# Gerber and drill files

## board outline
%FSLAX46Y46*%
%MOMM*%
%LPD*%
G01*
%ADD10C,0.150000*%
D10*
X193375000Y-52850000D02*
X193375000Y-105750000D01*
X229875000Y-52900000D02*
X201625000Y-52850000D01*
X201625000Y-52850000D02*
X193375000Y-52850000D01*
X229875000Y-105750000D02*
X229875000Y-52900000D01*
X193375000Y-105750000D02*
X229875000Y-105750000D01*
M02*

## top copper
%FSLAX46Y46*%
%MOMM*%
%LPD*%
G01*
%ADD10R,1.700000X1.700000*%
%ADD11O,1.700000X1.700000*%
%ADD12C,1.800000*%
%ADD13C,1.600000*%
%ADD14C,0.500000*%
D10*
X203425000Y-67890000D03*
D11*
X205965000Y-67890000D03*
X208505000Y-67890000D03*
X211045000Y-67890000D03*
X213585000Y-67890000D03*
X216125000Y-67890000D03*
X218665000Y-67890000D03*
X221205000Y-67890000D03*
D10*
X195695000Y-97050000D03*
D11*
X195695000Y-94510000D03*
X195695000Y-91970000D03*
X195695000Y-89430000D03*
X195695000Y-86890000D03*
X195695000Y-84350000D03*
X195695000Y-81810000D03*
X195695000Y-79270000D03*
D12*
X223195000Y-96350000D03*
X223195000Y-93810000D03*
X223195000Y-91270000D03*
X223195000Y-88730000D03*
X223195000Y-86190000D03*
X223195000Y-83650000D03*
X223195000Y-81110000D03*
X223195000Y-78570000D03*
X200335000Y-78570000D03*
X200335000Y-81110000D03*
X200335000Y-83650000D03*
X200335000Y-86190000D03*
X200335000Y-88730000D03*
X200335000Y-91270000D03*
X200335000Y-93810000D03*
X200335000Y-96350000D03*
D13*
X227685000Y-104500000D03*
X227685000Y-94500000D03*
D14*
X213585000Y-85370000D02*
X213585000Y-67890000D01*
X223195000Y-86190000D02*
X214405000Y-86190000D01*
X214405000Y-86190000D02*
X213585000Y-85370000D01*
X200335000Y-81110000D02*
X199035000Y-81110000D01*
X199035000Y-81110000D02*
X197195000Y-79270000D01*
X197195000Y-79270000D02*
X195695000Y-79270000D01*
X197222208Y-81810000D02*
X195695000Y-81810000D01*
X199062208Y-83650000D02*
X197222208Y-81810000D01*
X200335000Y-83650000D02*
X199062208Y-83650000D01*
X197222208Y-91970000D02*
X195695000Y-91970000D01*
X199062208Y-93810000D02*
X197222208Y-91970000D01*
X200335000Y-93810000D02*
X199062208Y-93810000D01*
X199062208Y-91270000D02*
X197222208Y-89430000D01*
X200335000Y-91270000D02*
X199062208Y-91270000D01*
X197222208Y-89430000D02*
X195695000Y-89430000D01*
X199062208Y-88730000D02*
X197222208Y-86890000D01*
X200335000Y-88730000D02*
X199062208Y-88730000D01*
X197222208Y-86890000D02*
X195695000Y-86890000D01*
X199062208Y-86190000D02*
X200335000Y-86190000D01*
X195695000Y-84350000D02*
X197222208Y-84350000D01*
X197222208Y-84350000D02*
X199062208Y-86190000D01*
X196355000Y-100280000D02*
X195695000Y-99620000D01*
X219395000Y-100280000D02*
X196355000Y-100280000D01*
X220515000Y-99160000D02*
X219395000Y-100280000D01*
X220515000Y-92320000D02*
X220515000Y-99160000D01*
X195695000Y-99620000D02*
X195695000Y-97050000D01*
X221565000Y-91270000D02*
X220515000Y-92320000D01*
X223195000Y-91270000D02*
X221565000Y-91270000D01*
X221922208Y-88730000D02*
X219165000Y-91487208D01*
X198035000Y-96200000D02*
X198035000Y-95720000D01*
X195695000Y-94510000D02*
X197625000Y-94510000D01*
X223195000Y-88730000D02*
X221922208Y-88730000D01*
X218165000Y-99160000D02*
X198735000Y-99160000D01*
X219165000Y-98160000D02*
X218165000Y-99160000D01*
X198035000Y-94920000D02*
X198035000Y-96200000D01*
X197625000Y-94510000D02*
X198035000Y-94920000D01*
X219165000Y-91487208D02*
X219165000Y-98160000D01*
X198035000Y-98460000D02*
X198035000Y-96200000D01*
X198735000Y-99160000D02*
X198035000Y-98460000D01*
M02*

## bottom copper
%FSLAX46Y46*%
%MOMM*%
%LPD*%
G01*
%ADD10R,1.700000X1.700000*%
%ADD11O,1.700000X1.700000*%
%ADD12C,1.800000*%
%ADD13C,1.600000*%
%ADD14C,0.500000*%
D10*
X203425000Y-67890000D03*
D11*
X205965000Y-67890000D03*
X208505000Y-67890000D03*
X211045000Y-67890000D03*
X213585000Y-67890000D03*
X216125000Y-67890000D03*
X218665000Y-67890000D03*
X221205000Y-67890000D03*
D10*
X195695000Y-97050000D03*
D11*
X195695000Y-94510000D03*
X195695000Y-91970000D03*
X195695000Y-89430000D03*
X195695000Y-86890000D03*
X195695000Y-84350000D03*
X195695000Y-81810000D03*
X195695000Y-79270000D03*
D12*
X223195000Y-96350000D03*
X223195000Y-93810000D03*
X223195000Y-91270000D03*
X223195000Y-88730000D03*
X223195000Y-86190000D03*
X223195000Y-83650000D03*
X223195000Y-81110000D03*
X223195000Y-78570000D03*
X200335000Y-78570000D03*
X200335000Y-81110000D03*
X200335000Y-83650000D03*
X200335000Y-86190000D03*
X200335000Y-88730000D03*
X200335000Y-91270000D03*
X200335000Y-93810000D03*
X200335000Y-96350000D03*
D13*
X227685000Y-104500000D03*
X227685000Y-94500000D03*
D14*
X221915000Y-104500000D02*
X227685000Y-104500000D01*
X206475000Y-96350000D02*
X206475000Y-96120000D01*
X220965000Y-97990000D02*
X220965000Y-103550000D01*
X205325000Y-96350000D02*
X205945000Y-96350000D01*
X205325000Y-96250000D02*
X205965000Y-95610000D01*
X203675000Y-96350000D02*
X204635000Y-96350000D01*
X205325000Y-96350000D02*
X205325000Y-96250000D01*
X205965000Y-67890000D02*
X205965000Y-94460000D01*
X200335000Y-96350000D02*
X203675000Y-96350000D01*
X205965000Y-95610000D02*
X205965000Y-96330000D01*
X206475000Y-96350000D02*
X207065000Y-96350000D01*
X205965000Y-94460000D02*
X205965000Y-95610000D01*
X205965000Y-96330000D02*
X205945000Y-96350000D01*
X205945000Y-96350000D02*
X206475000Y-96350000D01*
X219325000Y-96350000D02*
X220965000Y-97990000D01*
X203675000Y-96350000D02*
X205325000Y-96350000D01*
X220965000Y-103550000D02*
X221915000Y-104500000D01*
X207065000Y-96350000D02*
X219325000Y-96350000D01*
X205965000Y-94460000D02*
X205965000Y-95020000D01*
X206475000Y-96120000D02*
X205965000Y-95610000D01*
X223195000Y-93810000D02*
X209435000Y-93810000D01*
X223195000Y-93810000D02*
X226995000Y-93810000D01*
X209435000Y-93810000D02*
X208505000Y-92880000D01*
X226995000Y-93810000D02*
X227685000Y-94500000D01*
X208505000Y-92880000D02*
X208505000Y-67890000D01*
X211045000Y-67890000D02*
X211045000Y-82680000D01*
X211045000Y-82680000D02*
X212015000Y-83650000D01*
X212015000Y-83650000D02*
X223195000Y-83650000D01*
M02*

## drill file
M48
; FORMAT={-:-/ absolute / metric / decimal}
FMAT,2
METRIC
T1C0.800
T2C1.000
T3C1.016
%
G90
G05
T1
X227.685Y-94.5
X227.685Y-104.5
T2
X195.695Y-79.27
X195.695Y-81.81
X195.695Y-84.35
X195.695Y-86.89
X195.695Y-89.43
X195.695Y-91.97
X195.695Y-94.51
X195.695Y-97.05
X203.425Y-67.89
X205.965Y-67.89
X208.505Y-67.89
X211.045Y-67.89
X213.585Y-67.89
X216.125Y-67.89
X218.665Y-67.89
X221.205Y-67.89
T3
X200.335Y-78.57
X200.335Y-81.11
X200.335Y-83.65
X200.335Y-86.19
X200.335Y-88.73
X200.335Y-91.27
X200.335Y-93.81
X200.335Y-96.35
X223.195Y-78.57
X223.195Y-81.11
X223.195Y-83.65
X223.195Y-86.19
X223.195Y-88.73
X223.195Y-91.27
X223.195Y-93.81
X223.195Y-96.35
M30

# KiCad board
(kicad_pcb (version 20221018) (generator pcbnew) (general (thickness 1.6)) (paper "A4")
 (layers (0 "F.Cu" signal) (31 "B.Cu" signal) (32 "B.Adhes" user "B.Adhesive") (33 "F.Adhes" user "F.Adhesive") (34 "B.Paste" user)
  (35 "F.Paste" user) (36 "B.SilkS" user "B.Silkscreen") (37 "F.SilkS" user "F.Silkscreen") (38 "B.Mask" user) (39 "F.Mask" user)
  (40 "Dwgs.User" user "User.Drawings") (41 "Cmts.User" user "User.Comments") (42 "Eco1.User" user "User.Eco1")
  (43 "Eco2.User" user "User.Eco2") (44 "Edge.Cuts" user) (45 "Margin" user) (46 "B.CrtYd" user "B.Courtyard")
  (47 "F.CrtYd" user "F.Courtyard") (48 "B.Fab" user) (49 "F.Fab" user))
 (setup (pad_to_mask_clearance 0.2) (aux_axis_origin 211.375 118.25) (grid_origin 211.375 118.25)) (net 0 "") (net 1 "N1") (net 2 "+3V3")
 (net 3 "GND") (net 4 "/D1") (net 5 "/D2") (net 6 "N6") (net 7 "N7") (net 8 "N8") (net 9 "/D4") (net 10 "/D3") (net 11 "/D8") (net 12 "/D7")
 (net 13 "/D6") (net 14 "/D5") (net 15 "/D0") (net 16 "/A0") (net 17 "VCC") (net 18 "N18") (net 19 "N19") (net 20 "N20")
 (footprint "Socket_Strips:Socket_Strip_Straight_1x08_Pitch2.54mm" (layer "F.Cu") (at 203.425 67.89 90)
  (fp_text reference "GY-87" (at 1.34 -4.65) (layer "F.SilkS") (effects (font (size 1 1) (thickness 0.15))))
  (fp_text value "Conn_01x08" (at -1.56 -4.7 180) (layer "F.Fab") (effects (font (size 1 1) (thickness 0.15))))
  (pad "1" thru_hole rect (at 0 0 90) (size 1.7 1.7) (drill 1) (layers "*.Cu" "*.Mask") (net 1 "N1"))
  (pad "2" thru_hole oval (at 0 2.54 90) (size 1.7 1.7) (drill 1) (layers "*.Cu" "*.Mask") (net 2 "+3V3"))
  (pad "3" thru_hole oval (at 0 5.08 90) (size 1.7 1.7) (drill 1) (layers "*.Cu" "*.Mask") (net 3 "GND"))
  (pad "4" thru_hole oval (at 0 7.62 90) (size 1.7 1.7) (drill 1) (layers "*.Cu" "*.Mask") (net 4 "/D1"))
  (pad "5" thru_hole oval (at 0 10.16 90) (size 1.7 1.7) (drill 1) (layers "*.Cu" "*.Mask") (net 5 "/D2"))
  (pad "6" thru_hole oval (at 0 12.7 90) (size 1.7 1.7) (drill 1) (layers "*.Cu" "*.Mask") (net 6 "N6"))
  (pad "7" thru_hole oval (at 0 15.24 90) (size 1.7 1.7) (drill 1) (layers "*.Cu" "*.Mask") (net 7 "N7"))
  (pad "8" thru_hole oval (at 0 17.78 90) (size 1.7 1.7) (drill 1) (layers "*.Cu" "*.Mask") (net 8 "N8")))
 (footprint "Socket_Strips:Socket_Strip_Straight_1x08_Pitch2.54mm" (layer "F.Cu") (at 195.695 97.05 180)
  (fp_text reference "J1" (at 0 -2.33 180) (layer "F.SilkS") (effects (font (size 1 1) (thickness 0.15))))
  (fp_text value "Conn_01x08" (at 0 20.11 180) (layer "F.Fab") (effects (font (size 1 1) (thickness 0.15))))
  (pad "1" thru_hole rect (at 0 0 180) (size 1.7 1.7) (drill 1) (layers "*.Cu" "*.Mask") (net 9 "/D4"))
  (pad "2" thru_hole oval (at 0 2.54 180) (size 1.7 1.7) (drill 1) (layers "*.Cu" "*.Mask") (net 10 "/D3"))
  (pad "3" thru_hole oval (at 0 5.08 180) (size 1.7 1.7) (drill 1) (layers "*.Cu" "*.Mask") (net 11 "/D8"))
  (pad "4" thru_hole oval (at 0 7.62 180) (size 1.7 1.7) (drill 1) (layers "*.Cu" "*.Mask") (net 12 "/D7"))
  (pad "5" thru_hole oval (at 0 10.16 180) (size 1.7 1.7) (drill 1) (layers "*.Cu" "*.Mask") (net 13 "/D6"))
  (pad "6" thru_hole oval (at 0 12.7 180) (size 1.7 1.7) (drill 1) (layers "*.Cu" "*.Mask") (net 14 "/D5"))
  (pad "7" thru_hole oval (at 0 15.24 180) (size 1.7 1.7) (drill 1) (layers "*.Cu" "*.Mask") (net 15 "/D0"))
  (pad "8" thru_hole oval (at 0 17.78 180) (size 1.7 1.7) (drill 1) (layers "*.Cu" "*.Mask") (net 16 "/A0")))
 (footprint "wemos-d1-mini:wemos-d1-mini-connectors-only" (layer "F.Cu") (at 211.765 87.46 90)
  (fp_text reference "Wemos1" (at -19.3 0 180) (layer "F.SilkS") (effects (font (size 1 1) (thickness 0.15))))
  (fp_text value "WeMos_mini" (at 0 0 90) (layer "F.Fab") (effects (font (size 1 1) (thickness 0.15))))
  (pad "1" thru_hole circle (at -8.89 11.43 90) (size 1.8 1.8) (drill 1.016) (layers "*.Cu" "*.Mask") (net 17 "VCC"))
  (pad "2" thru_hole circle (at -6.35 11.43 90) (size 1.8 1.8) (drill 1.016) (layers "*.Cu" "*.Mask") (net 3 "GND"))
  (pad "3" thru_hole circle (at -3.81 11.43 90) (size 1.8 1.8) (drill 1.016) (layers "*.Cu" "*.Mask") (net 9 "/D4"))
  (pad "4" thru_hole circle (at -1.27 11.43 90) (size 1.8 1.8) (drill 1.016) (layers "*.Cu" "*.Mask") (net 10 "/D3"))
  (pad "5" thru_hole circle (at 1.27 11.43 90) (size 1.8 1.8) (drill 1.016) (layers "*.Cu" "*.Mask") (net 5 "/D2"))
  (pad "6" thru_hole circle (at 3.81 11.43 90) (size 1.8 1.8) (drill 1.016) (layers "*.Cu" "*.Mask") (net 4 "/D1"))
  (pad "7" thru_hole circle (at 6.35 11.43 90) (size 1.8 1.8) (drill 1.016) (layers "*.Cu" "*.Mask") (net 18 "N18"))
  (pad "8" thru_hole circle (at 8.89 11.43 90) (size 1.8 1.8) (drill 1.016) (layers "*.Cu" "*.Mask") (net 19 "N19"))
  (pad "9" thru_hole circle (at 8.89 -11.43 90) (size 1.8 1.8) (drill 1.016) (layers "*.Cu" "*.Mask") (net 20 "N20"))
  (pad "10" thru_hole circle (at 6.35 -11.43 90) (size 1.8 1.8) (drill 1.016) (layers "*.Cu" "*.Mask") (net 16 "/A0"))
  (pad "11" thru_hole circle (at 3.81 -11.43 90) (size 1.8 1.8) (drill 1.016) (layers "*.Cu" "*.Mask") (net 15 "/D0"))
  (pad "12" thru_hole circle (at 1.27 -11.43 90) (size 1.8 1.8) (drill 1.016) (layers "*.Cu" "*.Mask") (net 14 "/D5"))
  (pad "13" thru_hole circle (at -1.27 -11.43 90) (size 1.8 1.8) (drill 1.016) (layers "*.Cu" "*.Mask") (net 13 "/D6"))
  (pad "14" thru_hole circle (at -3.81 -11.43 90) (size 1.8 1.8) (drill 1.016) (layers "*.Cu" "*.Mask") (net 12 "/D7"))
  (pad "15" thru_hole circle (at -6.35 -11.43 90) (size 1.8 1.8) (drill 1.016) (layers "*.Cu" "*.Mask") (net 11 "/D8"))
  (pad "16" thru_hole circle (at -8.89 -11.43 90) (size 1.8 1.8) (drill 1.016) (layers "*.Cu" "*.Mask") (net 2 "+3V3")))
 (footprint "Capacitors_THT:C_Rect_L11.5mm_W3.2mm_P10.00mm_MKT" (layer "F.Cu") (at 227.685 104.5 90)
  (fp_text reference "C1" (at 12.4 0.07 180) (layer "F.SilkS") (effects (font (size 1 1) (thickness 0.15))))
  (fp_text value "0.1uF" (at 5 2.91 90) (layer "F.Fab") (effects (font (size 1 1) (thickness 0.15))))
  (pad "1" thru_hole circle (at 0 0 90) (size 1.6 1.6) (drill 0.8) (layers "*.Cu" "*.Mask") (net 2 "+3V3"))
  (pad "2" thru_hole circle (at 10 0 90) (size 1.6 1.6) (drill 0.8) (layers "*.Cu" "*.Mask") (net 3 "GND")))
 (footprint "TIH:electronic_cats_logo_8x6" (layer "F.Cu") (at 197.875 59.75)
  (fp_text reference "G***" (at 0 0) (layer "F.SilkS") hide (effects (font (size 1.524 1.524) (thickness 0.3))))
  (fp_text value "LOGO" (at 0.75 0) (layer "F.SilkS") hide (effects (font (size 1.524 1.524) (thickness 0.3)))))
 (gr_line (start 193.375 52.85) (end 193.375 105.75) (stroke (width 0.15) (type solid)) (layer "Edge.Cuts"))
 (gr_line (start 229.875 52.9) (end 201.625 52.85) (stroke (width 0.15) (type solid)) (layer "Edge.Cuts"))
 (gr_line (start 201.625 52.85) (end 193.375 52.85) (stroke (width 0.15) (type solid)) (layer "Edge.Cuts"))
 (gr_line (start 229.875 105.75) (end 229.875 52.9) (stroke (width 0.15) (type solid)) (layer "Edge.Cuts"))
 (gr_line (start 193.375 105.75) (end 229.875 105.75) (stroke (width 0.15) (type solid)) (layer "Edge.Cuts"))
 (segment (start 221.915 104.5) (end 227.685 104.5) (width 0.5) (layer "B.Cu") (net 2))
 (segment (start 206.475 96.35) (end 206.475 96.12) (width 0.5) (layer "B.Cu") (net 2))
 (segment (start 220.965 97.99) (end 220.965 103.55) (width 0.5) (layer "B.Cu") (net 2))
 (segment (start 205.325 96.35) (end 205.945 96.35) (width 0.5) (layer "B.Cu") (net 2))
 (segment (start 205.325 96.25) (end 205.965 95.61) (width 0.5) (layer "B.Cu") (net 2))
 (segment (start 203.675 96.35) (end 204.635 96.35) (width 0.5) (layer "B.Cu") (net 2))
 (segment (start 205.325 96.35) (end 205.325 96.25) (width 0.5) (layer "B.Cu") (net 2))
 (segment (start 205.965 67.89) (end 205.965 94.46) (width 0.5) (layer "B.Cu") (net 2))
 (segment (start 200.335 96.35) (end 203.675 96.35) (width 0.5) (layer "B.Cu") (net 2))
 (segment (start 205.965 95.61) (end 205.965 96.33) (width 0.5) (layer "B.Cu") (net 2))
 (segment (start 206.475 96.35) (end 207.065 96.35) (width 0.5) (layer "B.Cu") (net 2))
 (segment (start 205.965 94.46) (end 205.965 95.61) (width 0.5) (layer "B.Cu") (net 2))
 (segment (start 205.965 96.33) (end 205.945 96.35) (width 0.5) (layer "B.Cu") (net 2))
 (segment (start 205.945 96.35) (end 206.475 96.35) (width 0.5) (layer "B.Cu") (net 2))
 (segment (start 219.325 96.35) (end 220.965 97.99) (width 0.5) (layer "B.Cu") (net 2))
 (segment (start 203.675 96.35) (end 205.325 96.35) (width 0.5) (layer "B.Cu") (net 2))
 (segment (start 220.965 103.55) (end 221.915 104.5) (width 0.5) (layer "B.Cu") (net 2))
 (segment (start 207.065 96.35) (end 219.325 96.35) (width 0.5) (layer "B.Cu") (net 2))
 (segment (start 205.965 94.46) (end 205.965 95.02) (width 0.5) (layer "B.Cu") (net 2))
 (segment (start 206.475 96.12) (end 205.965 95.61) (width 0.5) (layer "B.Cu") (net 2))
 (segment (start 223.195 93.81) (end 209.435 93.81) (width 0.5) (layer "B.Cu") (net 3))
 (segment (start 223.195 93.81) (end 226.995 93.81) (width 0.5) (layer "B.Cu") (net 3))
 (segment (start 209.435 93.81) (end 208.505 92.88) (width 0.5) (layer "B.Cu") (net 3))
 (segment (start 226.995 93.81) (end 227.685 94.5) (width 0.5) (layer "B.Cu") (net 3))
 (segment (start 208.505 92.88) (end 208.505 67.89) (width 0.5) (layer "B.Cu") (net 3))
 (segment (start 211.045 67.89) (end 211.045 82.68) (width 0.5) (layer "B.Cu") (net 4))
 (segment (start 211.045 82.68) (end 212.015 83.65) (width 0.5) (layer "B.Cu") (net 4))
 (segment (start 212.015 83.65) (end 223.195 83.65) (width 0.5) (layer "B.Cu") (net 4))
 (segment (start 213.585 85.37) (end 213.585 67.89) (width 0.5) (layer "F.Cu") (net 5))
 (segment (start 223.195 86.19) (end 214.405 86.19) (width 0.5) (layer "F.Cu") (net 5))
 (segment (start 214.405 86.19) (end 213.585 85.37) (width 0.5) (layer "F.Cu") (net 5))
 (segment (start 200.335 81.11) (end 199.035 81.11) (width 0.5) (layer "F.Cu") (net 16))
 (segment (start 199.035 81.11) (end 197.195 79.27) (width 0.5) (layer "F.Cu") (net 16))
 (segment (start 197.195 79.27) (end 195.695 79.27) (width 0.5) (layer "F.Cu") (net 16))
 (segment (start 197.222208 81.81) (end 195.695 81.81) (width 0.5) (layer "F.Cu") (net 15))
 (segment (start 199.062208 83.65) (end 197.222208 81.81) (width 0.5) (layer "F.Cu") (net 15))
 (segment (start 200.335 83.65) (end 199.062208 83.65) (width 0.5) (layer "F.Cu") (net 15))
 (segment (start 197.222208 91.97) (end 195.695 91.97) (width 0.5) (layer "F.Cu") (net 11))
 (segment (start 199.062208 93.81) (end 197.222208 91.97) (width 0.5) (layer "F.Cu") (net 11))
 (segment (start 200.335 93.81) (end 199.062208 93.81) (width 0.5) (layer "F.Cu") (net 11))
 (segment (start 199.062208 91.27) (end 197.222208 89.43) (width 0.5) (layer "F.Cu") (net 12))
 (segment (start 200.335 91.27) (end 199.062208 91.27) (width 0.5) (layer "F.Cu") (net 12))
 (segment (start 197.222208 89.43) (end 195.695 89.43) (width 0.5) (layer "F.Cu") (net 12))
 (segment (start 199.062208 88.73) (end 197.222208 86.89) (width 0.5) (layer "F.Cu") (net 13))
 (segment (start 200.335 88.73) (end 199.062208 88.73) (width 0.5) (layer "F.Cu") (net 13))
 (segment (start 197.222208 86.89) (end 195.695 86.89) (width 0.5) (layer "F.Cu") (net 13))
 (segment (start 199.062208 86.19) (end 200.335 86.19) (width 0.5) (layer "F.Cu") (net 14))
 (segment (start 195.695 84.35) (end 197.222208 84.35) (width 0.5) (layer "F.Cu") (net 14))
 (segment (start 197.222208 84.35) (end 199.062208 86.19) (width 0.5) (layer "F.Cu") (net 14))
 (segment (start 196.355 100.28) (end 195.695 99.62) (width 0.5) (layer "F.Cu") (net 9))
 (segment (start 219.395 100.28) (end 196.355 100.28) (width 0.5) (layer "F.Cu") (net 9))
 (segment (start 220.515 99.16) (end 219.395 100.28) (width 0.5) (layer "F.Cu") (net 9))
 (segment (start 220.515 92.32) (end 220.515 99.16) (width 0.5) (layer "F.Cu") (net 9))
 (segment (start 195.695 99.62) (end 195.695 97.05) (width 0.5) (layer "F.Cu") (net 9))
 (segment (start 221.565 91.27) (end 220.515 92.32) (width 0.5) (layer "F.Cu") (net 9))
 (segment (start 223.195 91.27) (end 221.565 91.27) (width 0.5) (layer "F.Cu") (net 9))
 (segment (start 221.922208 88.73) (end 219.165 91.487208) (width 0.5) (layer "F.Cu") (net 10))
 (segment (start 198.035 96.2) (end 198.035 95.72) (width 0.5) (layer "F.Cu") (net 10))
 (segment (start 195.695 94.51) (end 197.625 94.51) (width 0.5) (layer "F.Cu") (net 10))
 (segment (start 223.195 88.73) (end 221.922208 88.73) (width 0.5) (layer "F.Cu") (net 10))
 (segment (start 218.165 99.16) (end 198.735 99.16) (width 0.5) (layer "F.Cu") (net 10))
 (segment (start 219.165 98.16) (end 218.165 99.16) (width 0.5) (layer "F.Cu") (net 10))
 (segment (start 198.035 94.92) (end 198.035 96.2) (width 0.5) (layer "F.Cu") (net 10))
 (segment (start 197.625 94.51) (end 198.035 94.92) (width 0.5) (layer "F.Cu") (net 10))
 (segment (start 219.165 91.487208) (end 219.165 98.16) (width 0.5) (layer "F.Cu") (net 10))
 (segment (start 198.035 98.46) (end 198.035 96.2) (width 0.5) (layer "F.Cu") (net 10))
 (segment (start 198.735 99.16) (end 198.035 98.46) (width 0.5) (layer "F.Cu") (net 10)))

